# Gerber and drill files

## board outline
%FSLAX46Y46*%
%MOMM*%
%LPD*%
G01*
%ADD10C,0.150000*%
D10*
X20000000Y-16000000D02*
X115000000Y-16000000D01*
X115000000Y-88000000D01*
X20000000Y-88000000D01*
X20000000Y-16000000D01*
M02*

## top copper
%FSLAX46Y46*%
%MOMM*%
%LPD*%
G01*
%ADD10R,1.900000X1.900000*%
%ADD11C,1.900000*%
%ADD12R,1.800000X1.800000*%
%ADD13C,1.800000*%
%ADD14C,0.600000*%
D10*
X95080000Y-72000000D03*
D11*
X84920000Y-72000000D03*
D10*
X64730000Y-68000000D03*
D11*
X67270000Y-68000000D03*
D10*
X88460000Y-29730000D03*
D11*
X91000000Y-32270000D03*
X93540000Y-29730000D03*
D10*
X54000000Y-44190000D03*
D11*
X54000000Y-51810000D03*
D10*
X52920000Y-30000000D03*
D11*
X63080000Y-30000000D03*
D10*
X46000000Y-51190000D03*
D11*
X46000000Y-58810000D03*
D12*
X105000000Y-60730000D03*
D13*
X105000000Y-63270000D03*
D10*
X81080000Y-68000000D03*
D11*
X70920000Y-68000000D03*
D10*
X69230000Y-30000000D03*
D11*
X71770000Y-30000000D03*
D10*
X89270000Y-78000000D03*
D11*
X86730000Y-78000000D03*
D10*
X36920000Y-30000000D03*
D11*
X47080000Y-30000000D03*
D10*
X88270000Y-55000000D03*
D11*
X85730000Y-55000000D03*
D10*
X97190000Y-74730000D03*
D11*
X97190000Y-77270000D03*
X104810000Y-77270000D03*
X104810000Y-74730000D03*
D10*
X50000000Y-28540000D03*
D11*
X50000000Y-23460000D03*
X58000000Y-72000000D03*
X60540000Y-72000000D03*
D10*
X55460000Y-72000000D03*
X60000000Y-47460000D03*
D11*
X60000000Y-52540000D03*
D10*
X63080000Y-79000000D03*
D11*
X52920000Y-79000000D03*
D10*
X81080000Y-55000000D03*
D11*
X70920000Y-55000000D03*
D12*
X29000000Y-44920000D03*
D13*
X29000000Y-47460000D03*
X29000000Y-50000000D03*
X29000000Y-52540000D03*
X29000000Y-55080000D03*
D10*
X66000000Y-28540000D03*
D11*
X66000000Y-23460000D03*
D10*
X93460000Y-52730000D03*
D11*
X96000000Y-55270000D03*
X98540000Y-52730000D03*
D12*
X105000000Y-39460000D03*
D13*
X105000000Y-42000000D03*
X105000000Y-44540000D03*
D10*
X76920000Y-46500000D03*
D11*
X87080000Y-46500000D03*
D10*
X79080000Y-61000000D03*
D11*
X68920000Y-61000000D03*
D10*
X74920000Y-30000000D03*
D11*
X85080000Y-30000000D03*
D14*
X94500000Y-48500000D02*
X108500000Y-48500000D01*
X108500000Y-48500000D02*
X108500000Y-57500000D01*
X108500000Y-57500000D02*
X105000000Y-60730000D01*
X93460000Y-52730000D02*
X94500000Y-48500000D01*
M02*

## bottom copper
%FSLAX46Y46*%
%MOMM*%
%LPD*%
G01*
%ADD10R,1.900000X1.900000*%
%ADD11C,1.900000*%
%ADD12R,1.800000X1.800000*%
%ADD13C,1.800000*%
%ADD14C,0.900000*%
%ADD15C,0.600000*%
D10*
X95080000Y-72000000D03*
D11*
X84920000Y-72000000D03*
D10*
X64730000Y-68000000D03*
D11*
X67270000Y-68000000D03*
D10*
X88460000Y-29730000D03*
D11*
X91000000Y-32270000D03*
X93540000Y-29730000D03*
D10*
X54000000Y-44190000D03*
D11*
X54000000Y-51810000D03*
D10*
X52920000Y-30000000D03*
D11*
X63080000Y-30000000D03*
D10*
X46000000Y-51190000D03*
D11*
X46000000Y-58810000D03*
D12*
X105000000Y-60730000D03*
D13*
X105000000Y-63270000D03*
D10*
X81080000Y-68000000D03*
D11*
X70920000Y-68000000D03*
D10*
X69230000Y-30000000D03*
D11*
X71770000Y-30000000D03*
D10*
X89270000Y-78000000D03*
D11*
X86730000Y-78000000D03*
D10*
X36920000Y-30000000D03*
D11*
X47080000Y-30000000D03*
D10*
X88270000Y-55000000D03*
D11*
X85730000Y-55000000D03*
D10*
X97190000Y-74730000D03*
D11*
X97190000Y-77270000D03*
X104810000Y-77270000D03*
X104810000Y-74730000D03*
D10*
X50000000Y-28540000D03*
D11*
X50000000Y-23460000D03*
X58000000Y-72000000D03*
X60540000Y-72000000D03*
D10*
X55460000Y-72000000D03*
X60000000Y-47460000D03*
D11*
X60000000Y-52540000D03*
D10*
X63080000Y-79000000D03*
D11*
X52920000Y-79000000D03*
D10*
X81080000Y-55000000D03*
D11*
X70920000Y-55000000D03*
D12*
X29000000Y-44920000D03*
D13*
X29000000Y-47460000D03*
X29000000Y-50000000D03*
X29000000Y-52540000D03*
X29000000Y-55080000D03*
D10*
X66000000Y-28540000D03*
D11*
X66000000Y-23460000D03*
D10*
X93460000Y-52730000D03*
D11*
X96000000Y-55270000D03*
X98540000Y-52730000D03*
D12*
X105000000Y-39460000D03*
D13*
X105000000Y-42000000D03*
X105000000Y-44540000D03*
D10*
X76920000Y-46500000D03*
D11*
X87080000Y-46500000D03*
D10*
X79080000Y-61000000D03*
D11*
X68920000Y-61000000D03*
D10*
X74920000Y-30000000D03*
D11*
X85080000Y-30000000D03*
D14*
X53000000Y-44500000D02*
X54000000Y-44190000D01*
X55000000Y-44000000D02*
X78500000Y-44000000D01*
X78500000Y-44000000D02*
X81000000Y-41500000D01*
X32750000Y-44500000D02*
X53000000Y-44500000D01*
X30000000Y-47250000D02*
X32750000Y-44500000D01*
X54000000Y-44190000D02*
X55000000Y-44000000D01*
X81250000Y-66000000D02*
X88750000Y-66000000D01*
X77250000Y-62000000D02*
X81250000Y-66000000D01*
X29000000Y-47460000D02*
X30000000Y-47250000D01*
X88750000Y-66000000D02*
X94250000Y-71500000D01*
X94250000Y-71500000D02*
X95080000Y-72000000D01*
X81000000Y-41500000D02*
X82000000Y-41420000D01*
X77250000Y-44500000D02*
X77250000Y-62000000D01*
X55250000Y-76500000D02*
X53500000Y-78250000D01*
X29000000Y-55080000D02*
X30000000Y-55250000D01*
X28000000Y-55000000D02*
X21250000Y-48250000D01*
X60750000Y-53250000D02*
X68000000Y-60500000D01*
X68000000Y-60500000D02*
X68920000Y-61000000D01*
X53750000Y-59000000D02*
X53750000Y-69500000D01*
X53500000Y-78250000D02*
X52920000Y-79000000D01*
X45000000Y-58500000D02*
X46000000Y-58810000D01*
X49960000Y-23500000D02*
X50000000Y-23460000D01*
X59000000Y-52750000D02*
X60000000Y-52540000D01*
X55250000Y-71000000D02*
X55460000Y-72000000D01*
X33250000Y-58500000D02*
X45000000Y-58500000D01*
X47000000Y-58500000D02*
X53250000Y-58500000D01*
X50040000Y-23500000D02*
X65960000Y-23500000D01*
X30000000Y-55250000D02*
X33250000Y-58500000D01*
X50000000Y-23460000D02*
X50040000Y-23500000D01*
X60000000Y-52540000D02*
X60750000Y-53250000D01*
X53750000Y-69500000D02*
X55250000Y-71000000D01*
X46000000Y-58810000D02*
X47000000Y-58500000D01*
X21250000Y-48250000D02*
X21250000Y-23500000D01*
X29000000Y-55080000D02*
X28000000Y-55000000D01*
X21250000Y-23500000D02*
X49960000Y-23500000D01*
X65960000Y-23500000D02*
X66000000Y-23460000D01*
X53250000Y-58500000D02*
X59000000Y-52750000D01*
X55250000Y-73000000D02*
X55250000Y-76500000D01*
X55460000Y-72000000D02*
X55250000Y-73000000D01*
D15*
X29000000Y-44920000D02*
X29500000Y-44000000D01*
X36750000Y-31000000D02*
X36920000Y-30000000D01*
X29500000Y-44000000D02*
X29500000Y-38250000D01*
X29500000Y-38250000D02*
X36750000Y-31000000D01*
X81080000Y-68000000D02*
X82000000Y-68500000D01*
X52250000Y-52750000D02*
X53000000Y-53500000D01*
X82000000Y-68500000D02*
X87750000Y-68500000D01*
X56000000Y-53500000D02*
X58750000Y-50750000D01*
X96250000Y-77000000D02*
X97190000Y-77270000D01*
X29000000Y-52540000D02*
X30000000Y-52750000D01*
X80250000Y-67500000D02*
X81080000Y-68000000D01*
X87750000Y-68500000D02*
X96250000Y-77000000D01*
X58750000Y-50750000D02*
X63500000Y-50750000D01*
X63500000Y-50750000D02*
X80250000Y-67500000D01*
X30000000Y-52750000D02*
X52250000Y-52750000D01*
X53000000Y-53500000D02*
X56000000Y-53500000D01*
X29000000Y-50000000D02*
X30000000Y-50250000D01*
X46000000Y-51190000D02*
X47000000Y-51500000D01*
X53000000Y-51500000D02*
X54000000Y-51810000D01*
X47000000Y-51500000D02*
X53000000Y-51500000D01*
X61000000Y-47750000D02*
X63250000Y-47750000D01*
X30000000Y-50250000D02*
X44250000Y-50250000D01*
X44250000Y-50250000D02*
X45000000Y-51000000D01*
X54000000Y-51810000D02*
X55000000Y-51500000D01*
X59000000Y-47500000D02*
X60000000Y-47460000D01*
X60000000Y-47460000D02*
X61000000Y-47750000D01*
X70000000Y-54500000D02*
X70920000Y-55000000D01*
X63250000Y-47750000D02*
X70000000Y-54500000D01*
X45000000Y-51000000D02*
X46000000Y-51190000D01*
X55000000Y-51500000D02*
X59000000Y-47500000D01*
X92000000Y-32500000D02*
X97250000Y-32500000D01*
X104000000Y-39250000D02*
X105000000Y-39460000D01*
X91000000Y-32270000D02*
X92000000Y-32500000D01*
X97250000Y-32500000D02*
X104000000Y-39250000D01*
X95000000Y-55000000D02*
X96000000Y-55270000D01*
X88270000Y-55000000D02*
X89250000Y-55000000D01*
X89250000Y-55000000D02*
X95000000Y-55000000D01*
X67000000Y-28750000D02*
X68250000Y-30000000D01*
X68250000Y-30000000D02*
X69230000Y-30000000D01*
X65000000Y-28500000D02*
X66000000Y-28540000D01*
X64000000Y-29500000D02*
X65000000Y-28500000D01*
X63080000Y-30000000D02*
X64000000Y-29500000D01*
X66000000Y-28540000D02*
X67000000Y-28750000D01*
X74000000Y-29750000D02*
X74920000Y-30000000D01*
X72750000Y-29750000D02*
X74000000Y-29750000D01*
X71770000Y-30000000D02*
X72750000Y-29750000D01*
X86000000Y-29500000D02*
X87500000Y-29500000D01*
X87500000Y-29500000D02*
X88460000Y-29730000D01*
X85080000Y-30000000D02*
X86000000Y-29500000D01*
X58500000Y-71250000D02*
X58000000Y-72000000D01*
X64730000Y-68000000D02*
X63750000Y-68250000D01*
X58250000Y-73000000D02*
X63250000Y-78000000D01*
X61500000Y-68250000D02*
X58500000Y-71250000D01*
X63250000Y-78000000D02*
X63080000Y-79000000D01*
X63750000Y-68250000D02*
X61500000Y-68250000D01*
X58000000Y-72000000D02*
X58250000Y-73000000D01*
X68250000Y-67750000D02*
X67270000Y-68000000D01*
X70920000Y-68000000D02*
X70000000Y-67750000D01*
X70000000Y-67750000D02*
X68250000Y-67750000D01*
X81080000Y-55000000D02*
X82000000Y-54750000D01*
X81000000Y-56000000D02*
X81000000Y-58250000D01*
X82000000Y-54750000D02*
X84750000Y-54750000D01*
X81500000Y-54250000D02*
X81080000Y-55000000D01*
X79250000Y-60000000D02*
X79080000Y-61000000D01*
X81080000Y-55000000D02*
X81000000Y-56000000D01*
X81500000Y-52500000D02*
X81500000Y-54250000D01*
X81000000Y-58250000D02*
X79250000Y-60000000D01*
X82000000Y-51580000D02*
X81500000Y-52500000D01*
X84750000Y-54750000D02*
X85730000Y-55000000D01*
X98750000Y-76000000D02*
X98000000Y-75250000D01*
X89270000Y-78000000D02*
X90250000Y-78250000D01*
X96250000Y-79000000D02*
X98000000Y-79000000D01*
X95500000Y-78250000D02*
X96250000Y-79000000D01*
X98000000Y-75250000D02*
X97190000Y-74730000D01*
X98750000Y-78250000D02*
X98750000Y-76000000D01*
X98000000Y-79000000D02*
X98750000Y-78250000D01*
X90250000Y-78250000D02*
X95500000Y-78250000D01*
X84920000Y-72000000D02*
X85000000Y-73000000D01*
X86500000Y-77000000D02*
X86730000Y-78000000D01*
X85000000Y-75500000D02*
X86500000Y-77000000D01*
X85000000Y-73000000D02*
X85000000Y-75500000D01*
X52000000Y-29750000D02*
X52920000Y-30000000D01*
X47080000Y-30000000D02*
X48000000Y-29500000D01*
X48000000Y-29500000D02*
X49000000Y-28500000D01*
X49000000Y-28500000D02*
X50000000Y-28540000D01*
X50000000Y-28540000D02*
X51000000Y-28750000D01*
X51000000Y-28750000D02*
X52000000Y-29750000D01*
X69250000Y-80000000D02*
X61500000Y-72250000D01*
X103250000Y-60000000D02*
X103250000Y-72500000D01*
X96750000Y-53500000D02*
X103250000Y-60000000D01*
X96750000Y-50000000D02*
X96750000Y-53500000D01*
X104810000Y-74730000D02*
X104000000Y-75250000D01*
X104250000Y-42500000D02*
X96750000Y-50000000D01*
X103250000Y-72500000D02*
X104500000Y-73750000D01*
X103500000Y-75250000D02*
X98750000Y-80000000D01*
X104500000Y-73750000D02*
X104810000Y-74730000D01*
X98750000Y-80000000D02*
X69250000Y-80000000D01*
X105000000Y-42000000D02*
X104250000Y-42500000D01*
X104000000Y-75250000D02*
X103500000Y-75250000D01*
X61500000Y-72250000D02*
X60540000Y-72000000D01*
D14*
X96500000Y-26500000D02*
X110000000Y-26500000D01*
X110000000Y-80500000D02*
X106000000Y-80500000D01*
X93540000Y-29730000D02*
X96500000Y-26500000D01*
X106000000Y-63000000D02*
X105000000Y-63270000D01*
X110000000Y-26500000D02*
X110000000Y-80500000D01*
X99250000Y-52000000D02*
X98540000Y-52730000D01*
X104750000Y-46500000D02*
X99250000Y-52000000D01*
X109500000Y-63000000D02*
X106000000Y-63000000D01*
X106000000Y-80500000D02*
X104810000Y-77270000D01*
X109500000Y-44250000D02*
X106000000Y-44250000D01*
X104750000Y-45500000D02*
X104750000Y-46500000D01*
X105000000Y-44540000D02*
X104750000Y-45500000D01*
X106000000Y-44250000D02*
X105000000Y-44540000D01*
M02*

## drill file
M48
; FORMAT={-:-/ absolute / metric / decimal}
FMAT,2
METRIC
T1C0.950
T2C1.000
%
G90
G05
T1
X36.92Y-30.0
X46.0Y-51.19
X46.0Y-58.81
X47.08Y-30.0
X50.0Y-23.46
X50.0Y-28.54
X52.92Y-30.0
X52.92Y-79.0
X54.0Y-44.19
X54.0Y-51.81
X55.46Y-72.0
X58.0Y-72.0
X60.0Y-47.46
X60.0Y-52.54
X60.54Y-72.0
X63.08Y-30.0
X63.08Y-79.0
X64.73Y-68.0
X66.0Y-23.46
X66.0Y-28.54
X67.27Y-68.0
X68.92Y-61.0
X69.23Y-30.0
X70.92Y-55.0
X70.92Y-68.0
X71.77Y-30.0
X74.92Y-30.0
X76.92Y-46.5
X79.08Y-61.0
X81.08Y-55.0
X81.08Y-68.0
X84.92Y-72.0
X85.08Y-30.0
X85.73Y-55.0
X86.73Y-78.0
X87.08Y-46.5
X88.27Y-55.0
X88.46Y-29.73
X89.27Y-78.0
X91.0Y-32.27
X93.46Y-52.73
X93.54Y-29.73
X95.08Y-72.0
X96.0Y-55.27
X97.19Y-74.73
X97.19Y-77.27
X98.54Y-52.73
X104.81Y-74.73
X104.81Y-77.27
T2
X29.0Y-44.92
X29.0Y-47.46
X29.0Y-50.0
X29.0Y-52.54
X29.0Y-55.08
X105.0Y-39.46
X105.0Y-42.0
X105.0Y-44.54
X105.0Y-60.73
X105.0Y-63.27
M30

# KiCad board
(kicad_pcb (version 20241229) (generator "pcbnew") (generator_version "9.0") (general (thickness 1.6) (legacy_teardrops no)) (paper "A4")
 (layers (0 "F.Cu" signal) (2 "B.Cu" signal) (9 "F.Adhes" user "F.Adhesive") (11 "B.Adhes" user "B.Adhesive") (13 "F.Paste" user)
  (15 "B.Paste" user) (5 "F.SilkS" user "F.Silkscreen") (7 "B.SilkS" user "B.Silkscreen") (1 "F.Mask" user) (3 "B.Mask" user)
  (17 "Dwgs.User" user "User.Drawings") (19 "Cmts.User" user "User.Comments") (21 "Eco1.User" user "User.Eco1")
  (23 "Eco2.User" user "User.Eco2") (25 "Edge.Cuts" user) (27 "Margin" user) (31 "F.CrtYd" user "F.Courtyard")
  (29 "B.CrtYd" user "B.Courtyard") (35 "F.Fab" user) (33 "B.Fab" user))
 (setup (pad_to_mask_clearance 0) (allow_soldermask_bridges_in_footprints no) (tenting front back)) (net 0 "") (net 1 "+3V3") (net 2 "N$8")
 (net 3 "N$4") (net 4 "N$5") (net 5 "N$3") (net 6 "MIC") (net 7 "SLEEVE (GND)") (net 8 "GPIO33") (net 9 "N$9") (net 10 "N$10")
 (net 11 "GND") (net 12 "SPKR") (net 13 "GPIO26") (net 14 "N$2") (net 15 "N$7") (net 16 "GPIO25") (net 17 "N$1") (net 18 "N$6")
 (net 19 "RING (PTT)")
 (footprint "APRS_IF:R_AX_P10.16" (layer "F.Cu") (at 90 72 180)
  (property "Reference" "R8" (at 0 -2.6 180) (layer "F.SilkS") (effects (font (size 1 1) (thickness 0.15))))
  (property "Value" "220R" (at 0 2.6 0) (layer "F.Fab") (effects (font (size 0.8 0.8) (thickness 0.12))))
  (pad "1" thru_hole rect (at -5.08 0 180) (size 1.9 1.9) (drill 0.95) (layers "*.Cu" "*.Mask") (remove_unused_layers no) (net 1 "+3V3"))
  (pad "2" thru_hole circle (at 5.08 0 180) (size 1.9 1.9) (drill 0.95) (layers "*.Cu" "*.Mask") (remove_unused_layers no) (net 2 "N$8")))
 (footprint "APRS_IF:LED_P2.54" (layer "F.Cu") (at 66 68)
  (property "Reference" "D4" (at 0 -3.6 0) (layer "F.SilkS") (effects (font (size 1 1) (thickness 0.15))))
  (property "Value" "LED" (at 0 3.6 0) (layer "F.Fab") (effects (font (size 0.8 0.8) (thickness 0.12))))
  (pad "1" thru_hole rect (at -1.27 0) (size 1.9 1.9) (drill 0.95) (layers "*.Cu" "*.Mask") (remove_unused_layers no) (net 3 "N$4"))
  (pad "2" thru_hole circle (at 1.27 0) (size 1.9 1.9) (drill 0.95) (layers "*.Cu" "*.Mask") (remove_unused_layers no) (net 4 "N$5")))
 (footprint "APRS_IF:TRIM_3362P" (layer "F.Cu") (at 91 31)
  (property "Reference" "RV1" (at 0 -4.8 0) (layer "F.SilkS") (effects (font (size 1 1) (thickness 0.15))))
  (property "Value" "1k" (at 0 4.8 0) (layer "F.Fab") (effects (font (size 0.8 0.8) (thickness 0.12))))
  (pad "1" thru_hole rect (at -2.54 -1.27) (size 1.9 1.9) (drill 0.95) (layers "*.Cu" "*.Mask") (remove_unused_layers no) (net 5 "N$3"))
  (pad "2" thru_hole circle (at 0 1.27) (size 1.9 1.9) (drill 0.95) (layers "*.Cu" "*.Mask") (remove_unused_layers no) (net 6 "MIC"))
  (pad "3" thru_hole circle (at 2.54 -1.27) (size 1.9 1.9) (drill 0.95) (layers "*.Cu" "*.Mask") (remove_unused_layers no)
   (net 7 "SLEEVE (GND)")))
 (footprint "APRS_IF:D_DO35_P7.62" (layer "F.Cu") (at 54 48 -90)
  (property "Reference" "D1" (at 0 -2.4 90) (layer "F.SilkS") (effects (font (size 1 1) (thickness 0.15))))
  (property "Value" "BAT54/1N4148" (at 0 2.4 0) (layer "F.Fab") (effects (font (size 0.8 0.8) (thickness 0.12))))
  (pad "1" thru_hole rect (at -3.81 0 270) (size 1.9 1.9) (drill 0.95) (layers "*.Cu" "*.Mask") (remove_unused_layers no) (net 1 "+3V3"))
  (pad "2" thru_hole circle (at 3.81 0 270) (size 1.9 1.9) (drill 0.95) (layers "*.Cu" "*.Mask") (remove_unused_layers no) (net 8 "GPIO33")))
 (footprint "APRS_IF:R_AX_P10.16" (layer "F.Cu") (at 58 30)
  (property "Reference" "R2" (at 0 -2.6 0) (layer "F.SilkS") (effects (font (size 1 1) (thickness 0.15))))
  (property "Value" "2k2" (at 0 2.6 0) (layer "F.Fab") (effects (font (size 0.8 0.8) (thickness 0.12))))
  (pad "1" thru_hole rect (at -5.08 0) (size 1.9 1.9) (drill 0.95) (layers "*.Cu" "*.Mask") (remove_unused_layers no) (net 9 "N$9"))
  (pad "2" thru_hole circle (at 5.08 0) (size 1.9 1.9) (drill 0.95) (layers "*.Cu" "*.Mask") (remove_unused_layers no) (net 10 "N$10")))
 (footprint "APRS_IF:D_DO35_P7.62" (layer "F.Cu") (at 46 55 -90)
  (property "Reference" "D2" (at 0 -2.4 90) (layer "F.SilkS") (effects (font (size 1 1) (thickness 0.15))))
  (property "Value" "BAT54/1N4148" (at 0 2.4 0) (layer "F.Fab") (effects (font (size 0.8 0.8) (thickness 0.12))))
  (pad "1" thru_hole rect (at -3.81 0 270) (size 1.9 1.9) (drill 0.95) (layers "*.Cu" "*.Mask") (remove_unused_layers no) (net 8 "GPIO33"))
  (pad "2" thru_hole circle (at 3.81 0 270) (size 1.9 1.9) (drill 0.95) (layers "*.Cu" "*.Mask") (remove_unused_layers no) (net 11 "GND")))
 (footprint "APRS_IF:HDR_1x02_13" (layer "F.Cu") (at 105 62)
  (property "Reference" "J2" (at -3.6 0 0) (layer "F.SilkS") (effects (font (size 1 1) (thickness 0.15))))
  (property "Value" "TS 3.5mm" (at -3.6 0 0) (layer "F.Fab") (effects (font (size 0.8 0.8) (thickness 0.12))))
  (pad "1" thru_hole rect (at 0 -1.27) (size 1.8 1.8) (drill 1) (layers "*.Cu" "*.Mask") (remove_unused_layers no) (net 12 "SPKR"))
  (pad "3" thru_hole circle (at 0 1.27) (size 1.8 1.8) (drill 1) (layers "*.Cu" "*.Mask") (remove_unused_layers no) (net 7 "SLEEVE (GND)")))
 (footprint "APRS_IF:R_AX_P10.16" (layer "F.Cu") (at 76 68 180)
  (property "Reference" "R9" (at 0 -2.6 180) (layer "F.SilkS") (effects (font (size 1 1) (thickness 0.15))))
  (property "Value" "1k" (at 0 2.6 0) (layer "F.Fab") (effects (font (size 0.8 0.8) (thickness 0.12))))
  (pad "1" thru_hole rect (at -5.08 0 180) (size 1.9 1.9) (drill 0.95) (layers "*.Cu" "*.Mask") (remove_unused_layers no) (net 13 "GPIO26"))
  (pad "2" thru_hole circle (at 5.08 0 180) (size 1.9 1.9) (drill 0.95) (layers "*.Cu" "*.Mask") (remove_unused_layers no) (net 4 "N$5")))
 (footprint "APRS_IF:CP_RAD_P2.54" (layer "F.Cu") (at 70.5 30)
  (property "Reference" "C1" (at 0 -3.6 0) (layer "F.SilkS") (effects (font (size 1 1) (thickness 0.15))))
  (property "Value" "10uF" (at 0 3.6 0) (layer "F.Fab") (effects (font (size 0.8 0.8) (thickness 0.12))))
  (pad "1" thru_hole rect (at -1.27 0) (size 1.9 1.9) (drill 0.95) (layers "*.Cu" "*.Mask") (remove_unused_layers no) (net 10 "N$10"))
  (pad "2" thru_hole circle (at 1.27 0) (size 1.9 1.9) (drill 0.95) (layers "*.Cu" "*.Mask") (remove_unused_layers no) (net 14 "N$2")))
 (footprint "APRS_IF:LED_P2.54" (layer "F.Cu") (at 88 78 180)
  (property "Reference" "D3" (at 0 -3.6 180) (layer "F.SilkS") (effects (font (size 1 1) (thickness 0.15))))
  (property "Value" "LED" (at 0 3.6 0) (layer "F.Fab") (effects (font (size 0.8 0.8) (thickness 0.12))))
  (pad "1" thru_hole rect (at -1.27 0 180) (size 1.9 1.9) (drill 0.95) (layers "*.Cu" "*.Mask") (remove_unused_layers no) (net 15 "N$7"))
  (pad "2" thru_hole circle (at 1.27 0 180) (size 1.9 1.9) (drill 0.95) (layers "*.Cu" "*.Mask") (remove_unused_layers no) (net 2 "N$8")))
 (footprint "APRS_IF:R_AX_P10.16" (layer "F.Cu") (at 42 30)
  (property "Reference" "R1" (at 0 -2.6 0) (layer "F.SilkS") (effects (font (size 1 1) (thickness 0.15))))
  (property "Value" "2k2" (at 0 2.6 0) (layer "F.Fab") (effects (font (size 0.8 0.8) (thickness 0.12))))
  (pad "1" thru_hole rect (at -5.08 0) (size 1.9 1.9) (drill 0.95) (layers "*.Cu" "*.Mask") (remove_unused_layers no) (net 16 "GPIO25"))
  (pad "2" thru_hole circle (at 5.08 0) (size 1.9 1.9) (drill 0.95) (layers "*.Cu" "*.Mask") (remove_unused_layers no) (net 9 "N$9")))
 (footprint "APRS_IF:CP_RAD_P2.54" (layer "F.Cu") (at 87 55 180)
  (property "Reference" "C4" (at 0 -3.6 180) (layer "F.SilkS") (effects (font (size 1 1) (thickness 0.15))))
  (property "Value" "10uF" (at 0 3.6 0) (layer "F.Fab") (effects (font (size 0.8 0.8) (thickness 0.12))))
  (pad "1" thru_hole rect (at -1.27 0 180) (size 1.9 1.9) (drill 0.95) (layers "*.Cu" "*.Mask") (remove_unused_layers no) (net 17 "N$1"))
  (pad "2" thru_hole circle (at 1.27 0 180) (size 1.9 1.9) (drill 0.95) (layers "*.Cu" "*.Mask") (remove_unused_layers no) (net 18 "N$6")))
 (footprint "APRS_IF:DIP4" (layer "F.Cu") (at 101 76)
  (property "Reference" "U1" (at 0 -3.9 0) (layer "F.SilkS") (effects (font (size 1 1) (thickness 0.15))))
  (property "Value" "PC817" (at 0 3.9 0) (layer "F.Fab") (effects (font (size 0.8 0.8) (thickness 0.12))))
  (pad "1" thru_hole rect (at -3.81 -1.27) (size 1.9 1.9) (drill 0.95) (layers "*.Cu" "*.Mask") (remove_unused_layers no) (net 15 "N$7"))
  (pad "2" thru_hole circle (at -3.81 1.27) (size 1.9 1.9) (drill 0.95) (layers "*.Cu" "*.Mask") (remove_unused_layers no) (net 13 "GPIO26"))
  (pad "3" thru_hole circle (at 3.81 1.27) (size 1.9 1.9) (drill 0.95) (layers "*.Cu" "*.Mask") (remove_unused_layers no)
   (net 7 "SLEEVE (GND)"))
  (pad "4" thru_hole circle (at 3.81 -1.27) (size 1.9 1.9) (drill 0.95) (layers "*.Cu" "*.Mask") (remove_unused_layers no)
   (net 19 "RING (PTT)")))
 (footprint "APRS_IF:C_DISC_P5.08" (layer "F.Cu") (at 50 26 90)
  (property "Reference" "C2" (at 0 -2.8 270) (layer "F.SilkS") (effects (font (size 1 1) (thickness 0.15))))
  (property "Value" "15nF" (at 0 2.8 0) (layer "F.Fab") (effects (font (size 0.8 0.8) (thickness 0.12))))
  (pad "1" thru_hole rect (at -2.54 0 90) (size 1.9 1.9) (drill 0.95) (layers "*.Cu" "*.Mask") (remove_unused_layers no) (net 9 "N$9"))
  (pad "2" thru_hole circle (at 2.54 0 90) (size 1.9 1.9) (drill 0.95) (layers "*.Cu" "*.Mask") (remove_unused_layers no) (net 11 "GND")))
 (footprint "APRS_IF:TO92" (layer "F.Cu") (at 58 72)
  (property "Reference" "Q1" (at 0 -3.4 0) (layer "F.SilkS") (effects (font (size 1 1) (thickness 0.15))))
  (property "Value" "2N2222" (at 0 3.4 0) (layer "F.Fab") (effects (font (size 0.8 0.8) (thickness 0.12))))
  (pad "1" thru_hole circle (at 0 0) (size 1.9 1.9) (drill 0.95) (layers "*.Cu" "*.Mask") (remove_unused_layers no) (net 3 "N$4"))
  (pad "2" thru_hole circle (at 2.54 0) (size 1.9 1.9) (drill 0.95) (layers "*.Cu" "*.Mask") (remove_unused_layers no) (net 19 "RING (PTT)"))
  (pad "3" thru_hole rect (at -2.54 0) (size 1.9 1.9) (drill 0.95) (layers "*.Cu" "*.Mask") (remove_unused_layers no) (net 11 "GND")))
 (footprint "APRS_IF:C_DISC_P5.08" (layer "F.Cu") (at 60 50 -90)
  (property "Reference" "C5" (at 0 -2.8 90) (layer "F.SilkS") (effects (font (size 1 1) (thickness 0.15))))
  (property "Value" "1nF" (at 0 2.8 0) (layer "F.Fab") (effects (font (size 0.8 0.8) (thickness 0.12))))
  (pad "1" thru_hole rect (at -2.54 0 270) (size 1.9 1.9) (drill 0.95) (layers "*.Cu" "*.Mask") (remove_unused_layers no) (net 8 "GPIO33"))
  (pad "2" thru_hole circle (at 2.54 0 270) (size 1.9 1.9) (drill 0.95) (layers "*.Cu" "*.Mask") (remove_unused_layers no) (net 11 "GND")))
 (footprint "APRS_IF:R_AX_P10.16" (layer "F.Cu") (at 58 79 180)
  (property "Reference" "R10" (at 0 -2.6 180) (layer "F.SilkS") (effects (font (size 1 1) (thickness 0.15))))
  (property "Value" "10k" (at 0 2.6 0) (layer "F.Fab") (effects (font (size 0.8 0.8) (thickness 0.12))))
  (pad "1" thru_hole rect (at -5.08 0 180) (size 1.9 1.9) (drill 0.95) (layers "*.Cu" "*.Mask") (remove_unused_layers no) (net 3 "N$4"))
  (pad "2" thru_hole circle (at 5.08 0 180) (size 1.9 1.9) (drill 0.95) (layers "*.Cu" "*.Mask") (remove_unused_layers no) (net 11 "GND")))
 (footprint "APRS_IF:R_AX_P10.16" (layer "F.Cu") (at 76 55 180)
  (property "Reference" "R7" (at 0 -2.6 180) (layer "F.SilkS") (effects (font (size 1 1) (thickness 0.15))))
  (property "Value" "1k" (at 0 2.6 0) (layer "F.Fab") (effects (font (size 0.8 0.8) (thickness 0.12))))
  (pad "1" thru_hole rect (at -5.08 0 180) (size 1.9 1.9) (drill 0.95) (layers "*.Cu" "*.Mask") (remove_unused_layers no) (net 18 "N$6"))
  (pad "2" thru_hole circle (at 5.08 0 180) (size 1.9 1.9) (drill 0.95) (layers "*.Cu" "*.Mask") (remove_unused_layers no) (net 8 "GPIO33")))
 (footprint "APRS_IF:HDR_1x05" (layer "F.Cu") (at 29 50)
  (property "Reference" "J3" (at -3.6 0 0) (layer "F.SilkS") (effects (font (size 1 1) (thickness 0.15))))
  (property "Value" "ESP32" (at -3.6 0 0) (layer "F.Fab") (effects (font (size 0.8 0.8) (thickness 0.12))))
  (pad "1" thru_hole rect (at 0 -5.08) (size 1.8 1.8) (drill 1) (layers "*.Cu" "*.Mask") (remove_unused_layers no) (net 16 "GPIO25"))
  (pad "2" thru_hole circle (at 0 -2.54) (size 1.8 1.8) (drill 1) (layers "*.Cu" "*.Mask") (remove_unused_layers no) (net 1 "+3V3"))
  (pad "3" thru_hole circle (at 0 0) (size 1.8 1.8) (drill 1) (layers "*.Cu" "*.Mask") (remove_unused_layers no) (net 8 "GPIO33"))
  (pad "4" thru_hole circle (at 0 2.54) (size 1.8 1.8) (drill 1) (layers "*.Cu" "*.Mask") (remove_unused_layers no) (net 13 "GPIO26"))
  (pad "5" thru_hole circle (at 0 5.08) (size 1.8 1.8) (drill 1) (layers "*.Cu" "*.Mask") (remove_unused_layers no) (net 11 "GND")))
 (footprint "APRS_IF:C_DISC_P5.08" (layer "F.Cu") (at 66 26 90)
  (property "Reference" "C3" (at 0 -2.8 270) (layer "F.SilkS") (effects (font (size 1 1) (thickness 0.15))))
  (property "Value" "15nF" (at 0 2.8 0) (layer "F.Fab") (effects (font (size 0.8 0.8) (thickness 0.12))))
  (pad "1" thru_hole rect (at -2.54 0 90) (size 1.9 1.9) (drill 0.95) (layers "*.Cu" "*.Mask") (remove_unused_layers no) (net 10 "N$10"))
  (pad "2" thru_hole circle (at 2.54 0 90) (size 1.9 1.9) (drill 0.95) (layers "*.Cu" "*.Mask") (remove_unused_layers no) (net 11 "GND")))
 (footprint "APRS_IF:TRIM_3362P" (layer "F.Cu") (at 96 54)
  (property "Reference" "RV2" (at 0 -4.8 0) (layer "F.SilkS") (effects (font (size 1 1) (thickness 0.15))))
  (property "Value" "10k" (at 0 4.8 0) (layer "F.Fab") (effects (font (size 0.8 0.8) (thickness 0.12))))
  (pad "1" thru_hole rect (at -2.54 -1.27) (size 1.9 1.9) (drill 0.95) (layers "*.Cu" "*.Mask") (remove_unused_layers no) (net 12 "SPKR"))
  (pad "2" thru_hole circle (at 0 1.27) (size 1.9 1.9) (drill 0.95) (layers "*.Cu" "*.Mask") (remove_unused_layers no) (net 17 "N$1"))
  (pad "3" thru_hole circle (at 2.54 -1.27) (size 1.9 1.9) (drill 0.95) (layers "*.Cu" "*.Mask") (remove_unused_layers no)
   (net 7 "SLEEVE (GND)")))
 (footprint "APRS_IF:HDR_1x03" (layer "F.Cu") (at 105 42)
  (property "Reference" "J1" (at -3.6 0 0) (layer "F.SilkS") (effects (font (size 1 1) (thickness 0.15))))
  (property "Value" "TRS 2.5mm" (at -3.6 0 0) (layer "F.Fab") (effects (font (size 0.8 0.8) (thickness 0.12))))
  (pad "1" thru_hole rect (at 0 -2.54) (size 1.8 1.8) (drill 1) (layers "*.Cu" "*.Mask") (remove_unused_layers no) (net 6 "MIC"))
  (pad "2" thru_hole circle (at 0 0) (size 1.8 1.8) (drill 1) (layers "*.Cu" "*.Mask") (remove_unused_layers no) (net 19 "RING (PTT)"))
  (pad "3" thru_hole circle (at 0 2.54) (size 1.8 1.8) (drill 1) (layers "*.Cu" "*.Mask") (remove_unused_layers no) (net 7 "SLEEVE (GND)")))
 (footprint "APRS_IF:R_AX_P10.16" (layer "F.Cu") (at 82 46.5)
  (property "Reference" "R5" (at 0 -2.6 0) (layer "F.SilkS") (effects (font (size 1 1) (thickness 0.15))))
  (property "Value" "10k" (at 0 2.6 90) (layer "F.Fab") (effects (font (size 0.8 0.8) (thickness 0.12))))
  (pad "1" thru_hole rect (at -5.08 0) (size 1.9 1.9) (drill 0.95) (layers "*.Cu" "*.Mask") (remove_unused_layers no) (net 1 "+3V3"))
  (pad "2" thru_hole circle (at 5.08 0) (size 1.9 1.9) (drill 0.95) (layers "*.Cu" "*.Mask") (remove_unused_layers no) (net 18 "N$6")))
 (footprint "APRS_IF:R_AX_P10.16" (layer "F.Cu") (at 74 61 180)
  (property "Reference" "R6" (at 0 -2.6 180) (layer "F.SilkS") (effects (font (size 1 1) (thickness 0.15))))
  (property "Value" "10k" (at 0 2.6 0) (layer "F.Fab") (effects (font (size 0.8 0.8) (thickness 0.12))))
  (pad "1" thru_hole rect (at -5.08 0 180) (size 1.9 1.9) (drill 0.95) (layers "*.Cu" "*.Mask") (remove_unused_layers no) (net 18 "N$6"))
  (pad "2" thru_hole circle (at 5.08 0 180) (size 1.9 1.9) (drill 0.95) (layers "*.Cu" "*.Mask") (remove_unused_layers no) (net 11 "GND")))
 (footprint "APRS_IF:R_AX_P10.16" (layer "F.Cu") (at 80 30)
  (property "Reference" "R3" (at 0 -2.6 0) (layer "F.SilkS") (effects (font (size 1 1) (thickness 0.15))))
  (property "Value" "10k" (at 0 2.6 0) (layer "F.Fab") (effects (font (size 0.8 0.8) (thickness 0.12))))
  (pad "1" thru_hole rect (at -5.08 0) (size 1.9 1.9) (drill 0.95) (layers "*.Cu" "*.Mask") (remove_unused_layers no) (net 14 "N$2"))
  (pad "2" thru_hole circle (at 5.08 0) (size 1.9 1.9) (drill 0.95) (layers "*.Cu" "*.Mask") (remove_unused_layers no) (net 5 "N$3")))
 (gr_rect (start 20 16) (end 115 88) (stroke (width 0.15) (type solid)) (fill no) (layer "Edge.Cuts"))
 (segment (start 53 44.5) (end 54 44.19) (width 0.9) (layer "B.Cu") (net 1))
 (segment (start 55 44) (end 78.5 44) (width 0.9) (layer "B.Cu") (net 1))
 (segment (start 78.5 44) (end 81 41.5) (width 0.9) (layer "B.Cu") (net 1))
 (segment (start 32.75 44.5) (end 53 44.5) (width 0.9) (layer "B.Cu") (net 1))
 (segment (start 30 47.25) (end 32.75 44.5) (width 0.9) (layer "B.Cu") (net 1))
 (segment (start 54 44.19) (end 55 44) (width 0.9) (layer "B.Cu") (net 1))
 (segment (start 81.25 66) (end 88.75 66) (width 0.9) (layer "B.Cu") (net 1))
 (segment (start 77.25 62) (end 81.25 66) (width 0.9) (layer "B.Cu") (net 1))
 (segment (start 29 47.46) (end 30 47.25) (width 0.9) (layer "B.Cu") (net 1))
 (segment (start 88.75 66) (end 94.25 71.5) (width 0.9) (layer "B.Cu") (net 1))
 (segment (start 94.25 71.5) (end 95.08 72) (width 0.9) (layer "B.Cu") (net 1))
 (segment (start 81 41.5) (end 82 41.42) (width 0.9) (layer "B.Cu") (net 1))
 (segment (start 77.25 44.5) (end 77.25 62) (width 0.9) (layer "B.Cu") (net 1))
 (segment (start 55.25 76.5) (end 53.5 78.25) (width 0.9) (layer "B.Cu") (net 11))
 (segment (start 29 55.08) (end 30 55.25) (width 0.9) (layer "B.Cu") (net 11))
 (segment (start 28 55) (end 21.25 48.25) (width 0.9) (layer "B.Cu") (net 11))
 (segment (start 60.75 53.25) (end 68 60.5) (width 0.9) (layer "B.Cu") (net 11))
 (segment (start 68 60.5) (end 68.92 61) (width 0.9) (layer "B.Cu") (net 11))
 (segment (start 53.75 59) (end 53.75 69.5) (width 0.9) (layer "B.Cu") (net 11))
 (segment (start 53.5 78.25) (end 52.92 79) (width 0.9) (layer "B.Cu") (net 11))
 (segment (start 45 58.5) (end 46 58.81) (width 0.9) (layer "B.Cu") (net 11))
 (segment (start 49.96 23.5) (end 50 23.46) (width 0.9) (layer "B.Cu") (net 11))
 (segment (start 59 52.75) (end 60 52.54) (width 0.9) (layer "B.Cu") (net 11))
 (segment (start 55.25 71) (end 55.46 72) (width 0.9) (layer "B.Cu") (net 11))
 (segment (start 33.25 58.5) (end 45 58.5) (width 0.9) (layer "B.Cu") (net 11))
 (segment (start 47 58.5) (end 53.25 58.5) (width 0.9) (layer "B.Cu") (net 11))
 (segment (start 50.04 23.5) (end 65.96 23.5) (width 0.9) (layer "B.Cu") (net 11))
 (segment (start 30 55.25) (end 33.25 58.5) (width 0.9) (layer "B.Cu") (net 11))
 (segment (start 50 23.46) (end 50.04 23.5) (width 0.9) (layer "B.Cu") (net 11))
 (segment (start 60 52.54) (end 60.75 53.25) (width 0.9) (layer "B.Cu") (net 11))
 (segment (start 53.75 69.5) (end 55.25 71) (width 0.9) (layer "B.Cu") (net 11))
 (segment (start 46 58.81) (end 47 58.5) (width 0.9) (layer "B.Cu") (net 11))
 (segment (start 21.25 48.25) (end 21.25 23.5) (width 0.9) (layer "B.Cu") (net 11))
 (segment (start 29 55.08) (end 28 55) (width 0.9) (layer "B.Cu") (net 11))
 (segment (start 21.25 23.5) (end 49.96 23.5) (width 0.9) (layer "B.Cu") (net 11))
 (segment (start 65.96 23.5) (end 66 23.46) (width 0.9) (layer "B.Cu") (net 11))
 (segment (start 53.25 58.5) (end 59 52.75) (width 0.9) (layer "B.Cu") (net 11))
 (segment (start 55.25 73) (end 55.25 76.5) (width 0.9) (layer "B.Cu") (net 11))
 (segment (start 55.46 72) (end 55.25 73) (width 0.9) (layer "B.Cu") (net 11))
 (segment (start 29 44.92) (end 29.5 44) (width 0.6) (layer "B.Cu") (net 16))
 (segment (start 36.75 31) (end 36.92 30) (width 0.6) (layer "B.Cu") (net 16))
 (segment (start 29.5 44) (end 29.5 38.25) (width 0.6) (layer "B.Cu") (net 16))
 (segment (start 29.5 38.25) (end 36.75 31) (width 0.6) (layer "B.Cu") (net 16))
 (segment (start 81.08 68) (end 82 68.5) (width 0.6) (layer "B.Cu") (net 13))
 (segment (start 52.25 52.75) (end 53 53.5) (width 0.6) (layer "B.Cu") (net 13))
 (segment (start 82 68.5) (end 87.75 68.5) (width 0.6) (layer "B.Cu") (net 13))
 (segment (start 56 53.5) (end 58.75 50.75) (width 0.6) (layer "B.Cu") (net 13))
 (segment (start 96.25 77) (end 97.19 77.27) (width 0.6) (layer "B.Cu") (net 13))
 (segment (start 29 52.54) (end 30 52.75) (width 0.6) (layer "B.Cu") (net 13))
 (segment (start 80.25 67.5) (end 81.08 68) (width 0.6) (layer "B.Cu") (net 13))
 (segment (start 87.75 68.5) (end 96.25 77) (width 0.6) (layer "B.Cu") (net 13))
 (segment (start 58.75 50.75) (end 63.5 50.75) (width 0.6) (layer "B.Cu") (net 13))
 (segment (start 63.5 50.75) (end 80.25 67.5) (width 0.6) (layer "B.Cu") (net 13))
 (segment (start 30 52.75) (end 52.25 52.75) (width 0.6) (layer "B.Cu") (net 13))
 (segment (start 53 53.5) (end 56 53.5) (width 0.6) (layer "B.Cu") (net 13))
 (segment (start 29 50) (end 30 50.25) (width 0.6) (layer "B.Cu") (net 8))
 (segment (start 46 51.19) (end 47 51.5) (width 0.6) (layer "B.Cu") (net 8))
 (segment (start 53 51.5) (end 54 51.81) (width 0.6) (layer "B.Cu") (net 8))
 (segment (start 47 51.5) (end 53 51.5) (width 0.6) (layer "B.Cu") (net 8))
 (segment (start 61 47.75) (end 63.25 47.75) (width 0.6) (layer "B.Cu") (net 8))
 (segment (start 30 50.25) (end 44.25 50.25) (width 0.6) (layer "B.Cu") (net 8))
 (segment (start 44.25 50.25) (end 45 51) (width 0.6) (layer "B.Cu") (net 8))
 (segment (start 54 51.81) (end 55 51.5) (width 0.6) (layer "B.Cu") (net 8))
 (segment (start 59 47.5) (end 60 47.46) (width 0.6) (layer "B.Cu") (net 8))
 (segment (start 60 47.46) (end 61 47.75) (width 0.6) (layer "B.Cu") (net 8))
 (segment (start 70 54.5) (end 70.92 55) (width 0.6) (layer "B.Cu") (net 8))
 (segment (start 63.25 47.75) (end 70 54.5) (width 0.6) (layer "B.Cu") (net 8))
 (segment (start 45 51) (end 46 51.19) (width 0.6) (layer "B.Cu") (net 8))
 (segment (start 55 51.5) (end 59 47.5) (width 0.6) (layer "B.Cu") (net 8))
 (segment (start 92 32.5) (end 97.25 32.5) (width 0.6) (layer "B.Cu") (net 6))
 (segment (start 104 39.25) (end 105 39.46) (width 0.6) (layer "B.Cu") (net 6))
 (segment (start 91 32.27) (end 92 32.5) (width 0.6) (layer "B.Cu") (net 6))
 (segment (start 97.25 32.5) (end 104 39.25) (width 0.6) (layer "B.Cu") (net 6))
 (segment (start 95 55) (end 96 55.27) (width 0.6) (layer "B.Cu") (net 17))
 (segment (start 88.27 55) (end 89.25 55) (width 0.6) (layer "B.Cu") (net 17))
 (segment (start 89.25 55) (end 95 55) (width 0.6) (layer "B.Cu") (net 17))
 (segment (start 67 28.75) (end 68.25 30) (width 0.6) (layer "B.Cu") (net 10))
 (segment (start 68.25 30) (end 69.23 30) (width 0.6) (layer "B.Cu") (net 10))
 (segment (start 65 28.5) (end 66 28.54) (width 0.6) (layer "B.Cu") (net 10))
 (segment (start 64 29.5) (end 65 28.5) (width 0.6) (layer "B.Cu") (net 10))
 (segment (start 63.08 30) (end 64 29.5) (width 0.6) (layer "B.Cu") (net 10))
 (segment (start 66 28.54) (end 67 28.75) (width 0.6) (layer "B.Cu") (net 10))
 (segment (start 74 29.75) (end 74.92 30) (width 0.6) (layer "B.Cu") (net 14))
 (segment (start 72.75 29.75) (end 74 29.75) (width 0.6) (layer "B.Cu") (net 14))
 (segment (start 71.77 30) (end 72.75 29.75) (width 0.6) (layer "B.Cu") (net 14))
 (segment (start 86 29.5) (end 87.5 29.5) (width 0.6) (layer "B.Cu") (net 5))
 (segment (start 87.5 29.5) (end 88.46 29.73) (width 0.6) (layer "B.Cu") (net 5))
 (segment (start 85.08 30) (end 86 29.5) (width 0.6) (layer "B.Cu") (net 5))
 (segment (start 58.5 71.25) (end 58 72) (width 0.6) (layer "B.Cu") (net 3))
 (segment (start 64.73 68) (end 63.75 68.25) (width 0.6) (layer "B.Cu") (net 3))
 (segment (start 58.25 73) (end 63.25 78) (width 0.6) (layer "B.Cu") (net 3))
 (segment (start 61.5 68.25) (end 58.5 71.25) (width 0.6) (layer "B.Cu") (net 3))
 (segment (start 63.25 78) (end 63.08 79) (width 0.6) (layer "B.Cu") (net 3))
 (segment (start 63.75 68.25) (end 61.5 68.25) (width 0.6) (layer "B.Cu") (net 3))
 (segment (start 58 72) (end 58.25 73) (width 0.6) (layer "B.Cu") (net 3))
 (segment (start 68.25 67.75) (end 67.27 68) (width 0.6) (layer "B.Cu") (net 4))
 (segment (start 70.92 68) (end 70 67.75) (width 0.6) (layer "B.Cu") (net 4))
 (segment (start 70 67.75) (end 68.25 67.75) (width 0.6) (layer "B.Cu") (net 4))
 (segment (start 81.08 55) (end 82 54.75) (width 0.6) (layer "B.Cu") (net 18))
 (segment (start 81 56) (end 81 58.25) (width 0.6) (layer "B.Cu") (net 18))
 (segment (start 82 54.75) (end 84.75 54.75) (width 0.6) (layer "B.Cu") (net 18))
 (segment (start 81.5 54.25) (end 81.08 55) (width 0.6) (layer "B.Cu") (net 18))
 (segment (start 79.25 60) (end 79.08 61) (width 0.6) (layer "B.Cu") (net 18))
 (segment (start 81.08 55) (end 81 56) (width 0.6) (layer "B.Cu") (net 18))
 (segment (start 81.5 52.5) (end 81.5 54.25) (width 0.6) (layer "B.Cu") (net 18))
 (segment (start 81 58.25) (end 79.25 60) (width 0.6) (layer "B.Cu") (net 18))
 (segment (start 82 51.58) (end 81.5 52.5) (width 0.6) (layer "B.Cu") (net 18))
 (segment (start 84.75 54.75) (end 85.73 55) (width 0.6) (layer "B.Cu") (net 18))
 (segment (start 98.75 76) (end 98 75.25) (width 0.6) (layer "B.Cu") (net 15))
 (segment (start 89.27 78) (end 90.25 78.25) (width 0.6) (layer "B.Cu") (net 15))
 (segment (start 96.25 79) (end 98 79) (width 0.6) (layer "B.Cu") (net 15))
 (segment (start 95.5 78.25) (end 96.25 79) (width 0.6) (layer "B.Cu") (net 15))
 (segment (start 98 75.25) (end 97.19 74.73) (width 0.6) (layer "B.Cu") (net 15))
 (segment (start 98.75 78.25) (end 98.75 76) (width 0.6) (layer "B.Cu") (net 15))
 (segment (start 98 79) (end 98.75 78.25) (width 0.6) (layer "B.Cu") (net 15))
 (segment (start 90.25 78.25) (end 95.5 78.25) (width 0.6) (layer "B.Cu") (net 15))
 (segment (start 84.92 72) (end 85 73) (width 0.6) (layer "B.Cu") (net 2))
 (segment (start 86.5 77) (end 86.73 78) (width 0.6) (layer "B.Cu") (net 2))
 (segment (start 85 75.5) (end 86.5 77) (width 0.6) (layer "B.Cu") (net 2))
 (segment (start 85 73) (end 85 75.5) (width 0.6) (layer "B.Cu") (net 2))
 (segment (start 52 29.75) (end 52.92 30) (width 0.6) (layer "B.Cu") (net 9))
 (segment (start 47.08 30) (end 48 29.5) (width 0.6) (layer "B.Cu") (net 9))
 (segment (start 48 29.5) (end 49 28.5) (width 0.6) (layer "B.Cu") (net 9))
 (segment (start 49 28.5) (end 50 28.54) (width 0.6) (layer "B.Cu") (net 9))
 (segment (start 50 28.54) (end 51 28.75) (width 0.6) (layer "B.Cu") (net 9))
 (segment (start 51 28.75) (end 52 29.75) (width 0.6) (layer "B.Cu") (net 9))
 (segment (start 69.25 80) (end 61.5 72.25) (width 0.6) (layer "B.Cu") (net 19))
 (segment (start 103.25 60) (end 103.25 72.5) (width 0.6) (layer "B.Cu") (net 19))
 (segment (start 96.75 53.5) (end 103.25 60) (width 0.6) (layer "B.Cu") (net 19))
 (segment (start 96.75 50) (end 96.75 53.5) (width 0.6) (layer "B.Cu") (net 19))
 (segment (start 104.81 74.73) (end 104 75.25) (width 0.6) (layer "B.Cu") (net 19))
 (segment (start 104.25 42.5) (end 96.75 50) (width 0.6) (layer "B.Cu") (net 19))
 (segment (start 103.25 72.5) (end 104.5 73.75) (width 0.6) (layer "B.Cu") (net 19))
 (segment (start 103.5 75.25) (end 98.75 80) (width 0.6) (layer "B.Cu") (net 19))
 (segment (start 104.5 73.75) (end 104.81 74.73) (width 0.6) (layer "B.Cu") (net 19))
 (segment (start 98.75 80) (end 69.25 80) (width 0.6) (layer "B.Cu") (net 19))
 (segment (start 105 42) (end 104.25 42.5) (width 0.6) (layer "B.Cu") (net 19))
 (segment (start 104 75.25) (end 103.5 75.25) (width 0.6) (layer "B.Cu") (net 19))
 (segment (start 61.5 72.25) (end 60.54 72) (width 0.6) (layer "B.Cu") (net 19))
 (segment (start 96.5 26.5) (end 110 26.5) (width 0.9) (layer "B.Cu") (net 7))
 (segment (start 110 80.5) (end 106 80.5) (width 0.9) (layer "B.Cu") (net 7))
 (segment (start 93.54 29.73) (end 96.5 26.5) (width 0.9) (layer "B.Cu") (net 7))
 (segment (start 106 63) (end 105 63.27) (width 0.9) (layer "B.Cu") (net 7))
 (segment (start 110 26.5) (end 110 80.5) (width 0.9) (layer "B.Cu") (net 7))
 (segment (start 99.25 52) (end 98.54 52.73) (width 0.9) (layer "B.Cu") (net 7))
 (segment (start 104.75 46.5) (end 99.25 52) (width 0.9) (layer "B.Cu") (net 7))
 (segment (start 109.5 63) (end 106 63) (width 0.9) (layer "B.Cu") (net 7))
 (segment (start 106 80.5) (end 104.81 77.27) (width 0.9) (layer "B.Cu") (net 7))
 (segment (start 109.5 44.25) (end 106 44.25) (width 0.9) (layer "B.Cu") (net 7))
 (segment (start 104.75 45.5) (end 104.75 46.5) (width 0.9) (layer "B.Cu") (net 7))
 (segment (start 105 44.54) (end 104.75 45.5) (width 0.9) (layer "B.Cu") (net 7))
 (segment (start 106 44.25) (end 105 44.54) (width 0.9) (layer "B.Cu") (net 7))
 (segment (start 94.5 48.5) (end 108.5 48.5) (width 0.6) (layer "F.Cu") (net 12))
 (segment (start 108.5 48.5) (end 108.5 57.5) (width 0.6) (layer "F.Cu") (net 12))
 (segment (start 108.5 57.5) (end 105 60.73) (width 0.6) (layer "F.Cu") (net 12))
 (segment (start 93.46 52.73) (end 94.5 48.5) (width 0.6) (layer "F.Cu") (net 12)))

